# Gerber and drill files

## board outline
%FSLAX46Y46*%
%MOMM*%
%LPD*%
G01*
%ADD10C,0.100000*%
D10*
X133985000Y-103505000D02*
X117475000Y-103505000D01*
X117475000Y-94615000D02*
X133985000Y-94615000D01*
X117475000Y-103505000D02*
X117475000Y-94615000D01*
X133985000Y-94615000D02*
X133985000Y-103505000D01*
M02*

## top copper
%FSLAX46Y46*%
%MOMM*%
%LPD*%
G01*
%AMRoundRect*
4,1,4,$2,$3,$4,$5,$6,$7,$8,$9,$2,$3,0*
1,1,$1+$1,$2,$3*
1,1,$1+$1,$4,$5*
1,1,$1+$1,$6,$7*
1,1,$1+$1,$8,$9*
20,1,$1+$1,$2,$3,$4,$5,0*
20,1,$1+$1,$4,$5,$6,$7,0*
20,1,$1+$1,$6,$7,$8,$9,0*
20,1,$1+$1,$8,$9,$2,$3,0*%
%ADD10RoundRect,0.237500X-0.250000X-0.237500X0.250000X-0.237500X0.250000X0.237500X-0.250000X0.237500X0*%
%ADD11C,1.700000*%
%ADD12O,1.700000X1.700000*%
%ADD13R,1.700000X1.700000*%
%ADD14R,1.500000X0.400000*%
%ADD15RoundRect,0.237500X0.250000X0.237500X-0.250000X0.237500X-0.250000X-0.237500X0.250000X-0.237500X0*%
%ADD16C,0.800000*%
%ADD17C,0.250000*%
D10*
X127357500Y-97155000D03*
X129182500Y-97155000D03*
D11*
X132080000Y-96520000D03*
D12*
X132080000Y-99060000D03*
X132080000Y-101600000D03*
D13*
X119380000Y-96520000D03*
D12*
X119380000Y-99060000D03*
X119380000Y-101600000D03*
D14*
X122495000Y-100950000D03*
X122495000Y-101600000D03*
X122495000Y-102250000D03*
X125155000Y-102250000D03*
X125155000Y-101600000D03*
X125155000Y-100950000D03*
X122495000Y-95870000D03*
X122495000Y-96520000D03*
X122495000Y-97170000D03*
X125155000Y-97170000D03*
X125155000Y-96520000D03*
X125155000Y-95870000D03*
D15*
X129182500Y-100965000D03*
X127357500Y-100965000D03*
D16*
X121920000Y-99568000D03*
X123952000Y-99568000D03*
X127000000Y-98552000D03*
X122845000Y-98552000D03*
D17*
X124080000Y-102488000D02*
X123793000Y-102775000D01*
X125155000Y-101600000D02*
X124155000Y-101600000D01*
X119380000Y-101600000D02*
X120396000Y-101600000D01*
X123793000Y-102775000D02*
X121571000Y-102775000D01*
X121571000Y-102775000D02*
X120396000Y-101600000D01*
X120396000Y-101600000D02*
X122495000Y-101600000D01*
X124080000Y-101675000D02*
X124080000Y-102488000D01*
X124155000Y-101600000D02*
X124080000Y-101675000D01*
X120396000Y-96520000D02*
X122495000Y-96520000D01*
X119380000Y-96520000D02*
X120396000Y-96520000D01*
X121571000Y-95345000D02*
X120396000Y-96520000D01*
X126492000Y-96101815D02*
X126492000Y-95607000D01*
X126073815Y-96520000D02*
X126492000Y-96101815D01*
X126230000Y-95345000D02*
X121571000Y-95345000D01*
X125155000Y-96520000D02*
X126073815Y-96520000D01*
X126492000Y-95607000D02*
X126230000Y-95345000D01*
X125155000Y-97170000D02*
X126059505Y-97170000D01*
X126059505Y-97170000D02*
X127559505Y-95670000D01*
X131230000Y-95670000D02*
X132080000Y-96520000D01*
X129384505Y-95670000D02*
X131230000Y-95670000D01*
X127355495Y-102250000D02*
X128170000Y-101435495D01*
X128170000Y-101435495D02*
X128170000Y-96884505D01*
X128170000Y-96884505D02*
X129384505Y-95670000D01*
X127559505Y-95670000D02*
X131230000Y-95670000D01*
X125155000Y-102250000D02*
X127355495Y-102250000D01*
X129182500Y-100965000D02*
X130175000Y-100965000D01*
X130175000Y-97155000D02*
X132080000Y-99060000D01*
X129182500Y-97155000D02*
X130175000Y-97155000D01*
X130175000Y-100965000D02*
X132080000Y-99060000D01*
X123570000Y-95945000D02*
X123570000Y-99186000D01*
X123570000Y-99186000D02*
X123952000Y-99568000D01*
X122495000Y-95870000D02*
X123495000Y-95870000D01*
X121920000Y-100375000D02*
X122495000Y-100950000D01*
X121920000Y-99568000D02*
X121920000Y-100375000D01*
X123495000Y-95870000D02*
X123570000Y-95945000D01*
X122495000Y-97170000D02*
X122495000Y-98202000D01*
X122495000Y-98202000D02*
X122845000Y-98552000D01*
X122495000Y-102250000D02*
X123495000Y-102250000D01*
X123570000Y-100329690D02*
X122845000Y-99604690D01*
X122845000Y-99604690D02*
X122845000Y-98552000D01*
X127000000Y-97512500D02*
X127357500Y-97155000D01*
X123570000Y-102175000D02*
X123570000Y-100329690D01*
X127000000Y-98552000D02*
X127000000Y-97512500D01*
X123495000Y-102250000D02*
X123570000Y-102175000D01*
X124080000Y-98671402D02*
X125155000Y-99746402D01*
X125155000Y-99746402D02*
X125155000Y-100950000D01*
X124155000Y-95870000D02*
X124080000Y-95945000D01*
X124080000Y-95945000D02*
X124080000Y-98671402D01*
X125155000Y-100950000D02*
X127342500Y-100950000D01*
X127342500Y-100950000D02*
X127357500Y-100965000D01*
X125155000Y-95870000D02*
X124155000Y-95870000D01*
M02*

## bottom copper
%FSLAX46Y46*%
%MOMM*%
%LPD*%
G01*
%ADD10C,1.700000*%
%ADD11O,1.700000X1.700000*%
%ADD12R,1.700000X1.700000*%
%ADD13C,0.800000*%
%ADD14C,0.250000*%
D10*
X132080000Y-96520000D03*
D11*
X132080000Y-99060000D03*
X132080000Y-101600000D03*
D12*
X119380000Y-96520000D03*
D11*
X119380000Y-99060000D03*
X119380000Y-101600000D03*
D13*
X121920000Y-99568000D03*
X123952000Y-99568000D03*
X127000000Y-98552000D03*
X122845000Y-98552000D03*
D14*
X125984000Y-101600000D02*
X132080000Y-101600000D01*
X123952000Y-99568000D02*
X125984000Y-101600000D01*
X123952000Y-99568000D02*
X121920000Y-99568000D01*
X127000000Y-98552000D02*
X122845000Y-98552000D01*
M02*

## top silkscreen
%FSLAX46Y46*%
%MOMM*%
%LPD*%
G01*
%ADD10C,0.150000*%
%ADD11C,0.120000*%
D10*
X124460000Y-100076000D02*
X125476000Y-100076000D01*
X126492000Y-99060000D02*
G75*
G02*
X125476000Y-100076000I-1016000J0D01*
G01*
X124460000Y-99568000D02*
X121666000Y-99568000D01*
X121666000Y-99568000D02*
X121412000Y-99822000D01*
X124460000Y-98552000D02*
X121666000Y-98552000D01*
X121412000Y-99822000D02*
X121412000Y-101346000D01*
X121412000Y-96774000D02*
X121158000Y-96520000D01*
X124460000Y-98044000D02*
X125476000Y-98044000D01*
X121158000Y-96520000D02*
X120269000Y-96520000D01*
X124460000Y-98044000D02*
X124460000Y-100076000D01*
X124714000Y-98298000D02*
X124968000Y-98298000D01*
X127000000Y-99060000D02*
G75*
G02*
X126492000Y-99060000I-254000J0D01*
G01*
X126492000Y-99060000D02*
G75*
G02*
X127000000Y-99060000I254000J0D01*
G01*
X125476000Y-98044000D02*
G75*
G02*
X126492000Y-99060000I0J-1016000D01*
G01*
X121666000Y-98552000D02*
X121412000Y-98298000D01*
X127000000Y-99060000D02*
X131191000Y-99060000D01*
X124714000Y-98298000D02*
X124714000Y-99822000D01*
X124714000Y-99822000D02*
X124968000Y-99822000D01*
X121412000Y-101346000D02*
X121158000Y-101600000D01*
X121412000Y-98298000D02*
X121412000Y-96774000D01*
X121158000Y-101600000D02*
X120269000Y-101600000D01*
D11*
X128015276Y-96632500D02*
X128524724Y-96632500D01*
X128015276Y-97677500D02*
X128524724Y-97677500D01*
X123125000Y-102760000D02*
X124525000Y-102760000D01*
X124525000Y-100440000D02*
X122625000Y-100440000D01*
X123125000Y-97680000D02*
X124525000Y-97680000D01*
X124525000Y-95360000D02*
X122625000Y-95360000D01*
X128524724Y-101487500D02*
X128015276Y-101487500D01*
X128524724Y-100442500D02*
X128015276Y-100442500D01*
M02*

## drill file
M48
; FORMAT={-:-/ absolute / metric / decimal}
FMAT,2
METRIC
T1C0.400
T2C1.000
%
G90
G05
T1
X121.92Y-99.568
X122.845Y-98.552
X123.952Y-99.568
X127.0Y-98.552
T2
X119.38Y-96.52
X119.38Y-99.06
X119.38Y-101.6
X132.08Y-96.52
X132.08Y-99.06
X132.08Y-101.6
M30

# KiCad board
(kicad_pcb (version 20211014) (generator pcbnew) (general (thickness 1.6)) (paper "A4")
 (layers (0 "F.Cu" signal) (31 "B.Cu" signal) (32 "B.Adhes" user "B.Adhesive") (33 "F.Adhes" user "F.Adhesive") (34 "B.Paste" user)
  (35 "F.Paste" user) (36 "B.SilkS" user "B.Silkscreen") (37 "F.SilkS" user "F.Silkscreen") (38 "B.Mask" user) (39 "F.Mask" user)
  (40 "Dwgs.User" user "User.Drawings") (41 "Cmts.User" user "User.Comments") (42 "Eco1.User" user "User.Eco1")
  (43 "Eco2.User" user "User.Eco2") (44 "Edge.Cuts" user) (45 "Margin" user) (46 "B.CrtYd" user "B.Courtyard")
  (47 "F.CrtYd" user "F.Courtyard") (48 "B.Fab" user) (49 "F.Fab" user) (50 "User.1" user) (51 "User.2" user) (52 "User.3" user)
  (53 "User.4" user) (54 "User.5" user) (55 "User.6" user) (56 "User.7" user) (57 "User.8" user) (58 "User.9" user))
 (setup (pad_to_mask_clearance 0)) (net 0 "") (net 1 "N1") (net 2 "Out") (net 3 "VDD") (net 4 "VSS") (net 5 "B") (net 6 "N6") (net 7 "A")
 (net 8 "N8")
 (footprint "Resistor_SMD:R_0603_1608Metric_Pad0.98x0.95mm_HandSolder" (layer "F.Cu") (at 128.27 97.155)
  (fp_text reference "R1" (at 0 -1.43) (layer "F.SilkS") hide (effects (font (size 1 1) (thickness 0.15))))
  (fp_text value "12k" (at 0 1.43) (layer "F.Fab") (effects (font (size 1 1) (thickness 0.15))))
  (fp_line (start -0.254724 -0.5225) (end 0.254724 -0.5225) (layer "F.SilkS") (width 0.12))
  (fp_line (start -0.254724 0.5225) (end 0.254724 0.5225) (layer "F.SilkS") (width 0.12))
  (pad "1" smd roundrect (at -0.9125 0) (size 0.975 0.95) (layers "F.Cu" "F.Paste" "F.Mask") (roundrect_rratio 0.25) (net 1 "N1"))
  (pad "2" smd roundrect (at 0.9125 0) (size 0.975 0.95) (layers "F.Cu" "F.Paste" "F.Mask") (roundrect_rratio 0.25) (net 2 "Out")))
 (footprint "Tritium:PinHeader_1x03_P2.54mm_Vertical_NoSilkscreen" (layer "F.Cu") (at 132.08 96.52)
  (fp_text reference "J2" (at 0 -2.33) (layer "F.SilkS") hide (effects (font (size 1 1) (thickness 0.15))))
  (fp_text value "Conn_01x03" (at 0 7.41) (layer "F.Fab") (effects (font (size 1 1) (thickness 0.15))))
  (pad "1" thru_hole circle (at 0 0) (size 1.7 1.7) (drill 1) (layers *.Cu *.Mask) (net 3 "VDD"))
  (pad "2" thru_hole oval (at 0 2.54) (size 1.7 1.7) (drill 1) (layers *.Cu *.Mask) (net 2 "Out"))
  (pad "3" thru_hole oval (at 0 5.08) (size 1.7 1.7) (drill 1) (layers *.Cu *.Mask) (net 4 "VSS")))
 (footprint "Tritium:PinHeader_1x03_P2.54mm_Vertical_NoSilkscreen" (layer "F.Cu") (at 119.38 96.52)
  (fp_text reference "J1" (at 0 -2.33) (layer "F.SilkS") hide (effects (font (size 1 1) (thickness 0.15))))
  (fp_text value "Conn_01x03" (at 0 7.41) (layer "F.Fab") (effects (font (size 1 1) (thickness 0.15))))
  (pad "1" thru_hole rect (at 0 0) (size 1.7 1.7) (drill 1) (layers *.Cu *.Mask) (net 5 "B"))
  (pad "2" thru_hole oval (at 0 2.54) (size 1.7 1.7) (drill 1) (layers *.Cu *.Mask) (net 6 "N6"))
  (pad "3" thru_hole oval (at 0 5.08) (size 1.7 1.7) (drill 1) (layers *.Cu *.Mask) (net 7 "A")))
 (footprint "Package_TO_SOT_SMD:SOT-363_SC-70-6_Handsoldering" (layer "F.Cu") (at 123.825 101.6)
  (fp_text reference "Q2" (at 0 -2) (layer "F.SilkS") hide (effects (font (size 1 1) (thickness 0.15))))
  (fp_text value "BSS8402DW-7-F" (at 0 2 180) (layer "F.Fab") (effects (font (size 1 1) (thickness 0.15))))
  (fp_line (start -0.7 1.16) (end 0.7 1.16) (layer "F.SilkS") (width 0.12))
  (fp_line (start 0.7 -1.16) (end -1.2 -1.16) (layer "F.SilkS") (width 0.12))
  (pad "1" smd rect (at -1.33 -0.65) (size 1.5 0.4) (layers "F.Cu" "F.Paste" "F.Mask") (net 4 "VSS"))
  (pad "2" smd rect (at -1.33 0) (size 1.5 0.4) (layers "F.Cu" "F.Paste" "F.Mask") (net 7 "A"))
  (pad "3" smd rect (at -1.33 0.65) (size 1.5 0.4) (layers "F.Cu" "F.Paste" "F.Mask") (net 1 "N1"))
  (pad "4" smd rect (at 1.33 0.65) (size 1.5 0.4) (layers "F.Cu" "F.Paste" "F.Mask") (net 3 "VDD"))
  (pad "5" smd rect (at 1.33 0) (size 1.5 0.4) (layers "F.Cu" "F.Paste" "F.Mask") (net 7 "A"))
  (pad "6" smd rect (at 1.33 -0.65) (size 1.5 0.4) (layers "F.Cu" "F.Paste" "F.Mask") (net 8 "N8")))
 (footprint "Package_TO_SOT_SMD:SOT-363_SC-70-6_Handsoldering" (layer "F.Cu") (at 123.825 96.52)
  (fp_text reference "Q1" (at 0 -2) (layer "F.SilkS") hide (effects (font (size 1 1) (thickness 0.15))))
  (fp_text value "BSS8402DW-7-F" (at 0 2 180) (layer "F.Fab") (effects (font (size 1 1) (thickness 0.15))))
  (fp_line (start -0.7 1.16) (end 0.7 1.16) (layer "F.SilkS") (width 0.12))
  (fp_line (start 0.7 -1.16) (end -1.2 -1.16) (layer "F.SilkS") (width 0.12))
  (pad "1" smd rect (at -1.33 -0.65) (size 1.5 0.4) (layers "F.Cu" "F.Paste" "F.Mask") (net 4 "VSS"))
  (pad "2" smd rect (at -1.33 0) (size 1.5 0.4) (layers "F.Cu" "F.Paste" "F.Mask") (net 5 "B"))
  (pad "3" smd rect (at -1.33 0.65) (size 1.5 0.4) (layers "F.Cu" "F.Paste" "F.Mask") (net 1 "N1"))
  (pad "4" smd rect (at 1.33 0.65) (size 1.5 0.4) (layers "F.Cu" "F.Paste" "F.Mask") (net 3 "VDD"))
  (pad "5" smd rect (at 1.33 0) (size 1.5 0.4) (layers "F.Cu" "F.Paste" "F.Mask") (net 5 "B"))
  (pad "6" smd rect (at 1.33 -0.65) (size 1.5 0.4) (layers "F.Cu" "F.Paste" "F.Mask") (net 8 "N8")))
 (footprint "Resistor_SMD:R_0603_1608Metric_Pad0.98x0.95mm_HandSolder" (layer "F.Cu") (at 128.27 100.965 180)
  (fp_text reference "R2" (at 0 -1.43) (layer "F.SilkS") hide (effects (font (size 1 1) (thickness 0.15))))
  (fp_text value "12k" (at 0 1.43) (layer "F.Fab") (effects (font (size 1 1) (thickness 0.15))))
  (fp_line (start -0.254724 -0.5225) (end 0.254724 -0.5225) (layer "F.SilkS") (width 0.12))
  (fp_line (start -0.254724 0.5225) (end 0.254724 0.5225) (layer "F.SilkS") (width 0.12))
  (pad "1" smd roundrect (at -0.9125 0 180) (size 0.975 0.95) (layers "F.Cu" "F.Paste" "F.Mask") (roundrect_rratio 0.25) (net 2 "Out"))
  (pad "2" smd roundrect (at 0.9125 0 180) (size 0.975 0.95) (layers "F.Cu" "F.Paste" "F.Mask") (roundrect_rratio 0.25) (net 8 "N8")))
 (gr_line (start 124.46 100.076) (end 125.476 100.076) (layer "F.SilkS") (width 0.15))
 (gr_arc (start 126.492 99.06) (mid 126.19442 99.77842) (end 125.476 100.076) (layer "F.SilkS") (width 0.15))
 (gr_line (start 124.46 99.568) (end 121.666 99.568) (layer "F.SilkS") (width 0.15))
 (gr_line (start 121.666 99.568) (end 121.412 99.822) (layer "F.SilkS") (width 0.15))
 (gr_line (start 124.46 98.552) (end 121.666 98.552) (layer "F.SilkS") (width 0.15))
 (gr_line (start 121.412 99.822) (end 121.412 101.346) (layer "F.SilkS") (width 0.15))
 (gr_line (start 121.412 96.774) (end 121.158 96.52) (layer "F.SilkS") (width 0.15))
 (gr_line (start 124.46 98.044) (end 125.476 98.044) (layer "F.SilkS") (width 0.15))
 (gr_line (start 121.158 96.52) (end 120.269 96.52) (layer "F.SilkS") (width 0.15))
 (gr_line (start 124.46 98.044) (end 124.46 100.076) (layer "F.SilkS") (width 0.15))
 (gr_line (start 124.714 98.298) (end 124.968 98.298) (layer "F.SilkS") (width 0.15))
 (gr_circle (center 126.746 99.06) (end 127 99.06) (layer "F.SilkS") (width 0.15) (fill none))
 (gr_arc (start 125.476 98.044) (mid 126.19442 98.34158) (end 126.492 99.06) (layer "F.SilkS") (width 0.15))
 (gr_line (start 121.666 98.552) (end 121.412 98.298) (layer "F.SilkS") (width 0.15))
 (gr_line (start 127 99.06) (end 131.191 99.06) (layer "F.SilkS") (width 0.15))
 (gr_line (start 124.714 98.298) (end 124.714 99.822) (layer "F.SilkS") (width 0.15))
 (gr_line (start 124.714 99.822) (end 124.968 99.822) (layer "F.SilkS") (width 0.15))
 (gr_line (start 121.412 101.346) (end 121.158 101.6) (layer "F.SilkS") (width 0.15))
 (gr_line (start 121.412 98.298) (end 121.412 96.774) (layer "F.SilkS") (width 0.15))
 (gr_line (start 121.158 101.6) (end 120.269 101.6) (layer "F.SilkS") (width 0.15))
 (gr_line (start 133.985 103.505) (end 117.475 103.505) (layer "Edge.Cuts") (width 0.1))
 (gr_line (start 117.475 94.615) (end 133.985 94.615) (layer "Edge.Cuts") (width 0.1))
 (gr_line (start 117.475 103.505) (end 117.475 94.615) (layer "Edge.Cuts") (width 0.1))
 (gr_line (start 133.985 94.615) (end 133.985 103.505) (layer "Edge.Cuts") (width 0.1))
 (segment (start 124.08 102.488) (end 123.793 102.775) (width 0.25) (layer "F.Cu") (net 7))
 (segment (start 125.155 101.6) (end 124.155 101.6) (width 0.25) (layer "F.Cu") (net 7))
 (segment (start 119.38 101.6) (end 120.396 101.6) (width 0.25) (layer "F.Cu") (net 7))
 (segment (start 123.793 102.775) (end 121.571 102.775) (width 0.25) (layer "F.Cu") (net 7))
 (segment (start 121.571 102.775) (end 120.396 101.6) (width 0.25) (layer "F.Cu") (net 7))
 (segment (start 120.396 101.6) (end 122.495 101.6) (width 0.25) (layer "F.Cu") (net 7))
 (segment (start 124.08 101.675) (end 124.08 102.488) (width 0.25) (layer "F.Cu") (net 7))
 (segment (start 124.155 101.6) (end 124.08 101.675) (width 0.25) (layer "F.Cu") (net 7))
 (segment (start 120.396 96.52) (end 122.495 96.52) (width 0.25) (layer "F.Cu") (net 5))
 (segment (start 119.38 96.52) (end 120.396 96.52) (width 0.25) (layer "F.Cu") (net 5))
 (segment (start 121.571 95.345) (end 120.396 96.52) (width 0.25) (layer "F.Cu") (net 5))
 (segment (start 126.492 96.101815) (end 126.492 95.607) (width 0.25) (layer "F.Cu") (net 5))
 (segment (start 126.073815 96.52) (end 126.492 96.101815) (width 0.25) (layer "F.Cu") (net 5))
 (segment (start 126.23 95.345) (end 121.571 95.345) (width 0.25) (layer "F.Cu") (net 5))
 (segment (start 125.155 96.52) (end 126.073815 96.52) (width 0.25) (layer "F.Cu") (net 5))
 (segment (start 126.492 95.607) (end 126.23 95.345) (width 0.25) (layer "F.Cu") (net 5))
 (segment (start 125.155 97.17) (end 126.059505 97.17) (width 0.25) (layer "F.Cu") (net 3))
 (segment (start 126.059505 97.17) (end 127.559505 95.67) (width 0.25) (layer "F.Cu") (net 3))
 (segment (start 131.23 95.67) (end 132.08 96.52) (width 0.25) (layer "F.Cu") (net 3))
 (segment (start 129.384505 95.67) (end 131.23 95.67) (width 0.25) (layer "F.Cu") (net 3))
 (segment (start 127.355495 102.25) (end 128.17 101.435495) (width 0.25) (layer "F.Cu") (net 3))
 (segment (start 128.17 101.435495) (end 128.17 96.884505) (width 0.25) (layer "F.Cu") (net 3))
 (segment (start 128.17 96.884505) (end 129.384505 95.67) (width 0.25) (layer "F.Cu") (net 3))
 (segment (start 127.559505 95.67) (end 131.23 95.67) (width 0.25) (layer "F.Cu") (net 3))
 (segment (start 125.155 102.25) (end 127.355495 102.25) (width 0.25) (layer "F.Cu") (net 3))
 (segment (start 129.1825 100.965) (end 130.175 100.965) (width 0.25) (layer "F.Cu") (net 2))
 (segment (start 130.175 97.155) (end 132.08 99.06) (width 0.25) (layer "F.Cu") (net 2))
 (segment (start 129.1825 97.155) (end 130.175 97.155) (width 0.25) (layer "F.Cu") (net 2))
 (segment (start 130.175 100.965) (end 132.08 99.06) (width 0.25) (layer "F.Cu") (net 2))
 (segment (start 123.57 95.945) (end 123.57 99.186) (width 0.25) (layer "F.Cu") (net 4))
 (segment (start 123.57 99.186) (end 123.952 99.568) (width 0.25) (layer "F.Cu") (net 4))
 (segment (start 122.495 95.87) (end 123.495 95.87) (width 0.25) (layer "F.Cu") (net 4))
 (segment (start 121.92 100.375) (end 122.495 100.95) (width 0.25) (layer "F.Cu") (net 4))
 (segment (start 121.92 99.568) (end 121.92 100.375) (width 0.25) (layer "F.Cu") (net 4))
 (segment (start 123.495 95.87) (end 123.57 95.945) (width 0.25) (layer "F.Cu") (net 4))
 (via (at 121.92 99.568) (size 0.8) (drill 0.4) (layers "F.Cu" "B.Cu") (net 4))
 (via (at 123.952 99.568) (size 0.8) (drill 0.4) (layers "F.Cu" "B.Cu") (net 4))
 (segment (start 125.984 101.6) (end 132.08 101.6) (width 0.25) (layer "B.Cu") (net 4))
 (segment (start 123.952 99.568) (end 125.984 101.6) (width 0.25) (layer "B.Cu") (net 4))
 (segment (start 123.952 99.568) (end 121.92 99.568) (width 0.25) (layer "B.Cu") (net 4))
 (segment (start 122.495 97.17) (end 122.495 98.202) (width 0.25) (layer "F.Cu") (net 1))
 (segment (start 122.495 98.202) (end 122.845 98.552) (width 0.25) (layer "F.Cu") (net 1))
 (segment (start 122.495 102.25) (end 123.495 102.25) (width 0.25) (layer "F.Cu") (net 1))
 (segment (start 123.57 100.32969) (end 122.845 99.60469) (width 0.25) (layer "F.Cu") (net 1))
 (segment (start 122.845 99.60469) (end 122.845 98.552) (width 0.25) (layer "F.Cu") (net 1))
 (segment (start 127 97.5125) (end 127.3575 97.155) (width 0.25) (layer "F.Cu") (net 1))
 (segment (start 123.57 102.175) (end 123.57 100.32969) (width 0.25) (layer "F.Cu") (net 1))
 (segment (start 127 98.552) (end 127 97.5125) (width 0.25) (layer "F.Cu") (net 1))
 (segment (start 123.495 102.25) (end 123.57 102.175) (width 0.25) (layer "F.Cu") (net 1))
 (via (at 127 98.552) (size 0.8) (drill 0.4) (layers "F.Cu" "B.Cu") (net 1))
 (via (at 122.845 98.552) (size 0.8) (drill 0.4) (layers "F.Cu" "B.Cu") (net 1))
 (segment (start 127 98.552) (end 122.845 98.552) (width 0.25) (layer "B.Cu") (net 1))
 (segment (start 124.08 98.671402) (end 125.155 99.746402) (width 0.25) (layer "F.Cu") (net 8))
 (segment (start 125.155 99.746402) (end 125.155 100.95) (width 0.25) (layer "F.Cu") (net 8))
 (segment (start 124.155 95.87) (end 124.08 95.945) (width 0.25) (layer "F.Cu") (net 8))
 (segment (start 124.08 95.945) (end 124.08 98.671402) (width 0.25) (layer "F.Cu") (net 8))
 (segment (start 125.155 100.95) (end 127.3425 100.95) (width 0.25) (layer "F.Cu") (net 8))
 (segment (start 127.3425 100.95) (end 127.3575 100.965) (width 0.25) (layer "F.Cu") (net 8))
 (segment (start 125.155 95.87) (end 124.155 95.87) (width 0.25) (layer "F.Cu") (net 8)))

